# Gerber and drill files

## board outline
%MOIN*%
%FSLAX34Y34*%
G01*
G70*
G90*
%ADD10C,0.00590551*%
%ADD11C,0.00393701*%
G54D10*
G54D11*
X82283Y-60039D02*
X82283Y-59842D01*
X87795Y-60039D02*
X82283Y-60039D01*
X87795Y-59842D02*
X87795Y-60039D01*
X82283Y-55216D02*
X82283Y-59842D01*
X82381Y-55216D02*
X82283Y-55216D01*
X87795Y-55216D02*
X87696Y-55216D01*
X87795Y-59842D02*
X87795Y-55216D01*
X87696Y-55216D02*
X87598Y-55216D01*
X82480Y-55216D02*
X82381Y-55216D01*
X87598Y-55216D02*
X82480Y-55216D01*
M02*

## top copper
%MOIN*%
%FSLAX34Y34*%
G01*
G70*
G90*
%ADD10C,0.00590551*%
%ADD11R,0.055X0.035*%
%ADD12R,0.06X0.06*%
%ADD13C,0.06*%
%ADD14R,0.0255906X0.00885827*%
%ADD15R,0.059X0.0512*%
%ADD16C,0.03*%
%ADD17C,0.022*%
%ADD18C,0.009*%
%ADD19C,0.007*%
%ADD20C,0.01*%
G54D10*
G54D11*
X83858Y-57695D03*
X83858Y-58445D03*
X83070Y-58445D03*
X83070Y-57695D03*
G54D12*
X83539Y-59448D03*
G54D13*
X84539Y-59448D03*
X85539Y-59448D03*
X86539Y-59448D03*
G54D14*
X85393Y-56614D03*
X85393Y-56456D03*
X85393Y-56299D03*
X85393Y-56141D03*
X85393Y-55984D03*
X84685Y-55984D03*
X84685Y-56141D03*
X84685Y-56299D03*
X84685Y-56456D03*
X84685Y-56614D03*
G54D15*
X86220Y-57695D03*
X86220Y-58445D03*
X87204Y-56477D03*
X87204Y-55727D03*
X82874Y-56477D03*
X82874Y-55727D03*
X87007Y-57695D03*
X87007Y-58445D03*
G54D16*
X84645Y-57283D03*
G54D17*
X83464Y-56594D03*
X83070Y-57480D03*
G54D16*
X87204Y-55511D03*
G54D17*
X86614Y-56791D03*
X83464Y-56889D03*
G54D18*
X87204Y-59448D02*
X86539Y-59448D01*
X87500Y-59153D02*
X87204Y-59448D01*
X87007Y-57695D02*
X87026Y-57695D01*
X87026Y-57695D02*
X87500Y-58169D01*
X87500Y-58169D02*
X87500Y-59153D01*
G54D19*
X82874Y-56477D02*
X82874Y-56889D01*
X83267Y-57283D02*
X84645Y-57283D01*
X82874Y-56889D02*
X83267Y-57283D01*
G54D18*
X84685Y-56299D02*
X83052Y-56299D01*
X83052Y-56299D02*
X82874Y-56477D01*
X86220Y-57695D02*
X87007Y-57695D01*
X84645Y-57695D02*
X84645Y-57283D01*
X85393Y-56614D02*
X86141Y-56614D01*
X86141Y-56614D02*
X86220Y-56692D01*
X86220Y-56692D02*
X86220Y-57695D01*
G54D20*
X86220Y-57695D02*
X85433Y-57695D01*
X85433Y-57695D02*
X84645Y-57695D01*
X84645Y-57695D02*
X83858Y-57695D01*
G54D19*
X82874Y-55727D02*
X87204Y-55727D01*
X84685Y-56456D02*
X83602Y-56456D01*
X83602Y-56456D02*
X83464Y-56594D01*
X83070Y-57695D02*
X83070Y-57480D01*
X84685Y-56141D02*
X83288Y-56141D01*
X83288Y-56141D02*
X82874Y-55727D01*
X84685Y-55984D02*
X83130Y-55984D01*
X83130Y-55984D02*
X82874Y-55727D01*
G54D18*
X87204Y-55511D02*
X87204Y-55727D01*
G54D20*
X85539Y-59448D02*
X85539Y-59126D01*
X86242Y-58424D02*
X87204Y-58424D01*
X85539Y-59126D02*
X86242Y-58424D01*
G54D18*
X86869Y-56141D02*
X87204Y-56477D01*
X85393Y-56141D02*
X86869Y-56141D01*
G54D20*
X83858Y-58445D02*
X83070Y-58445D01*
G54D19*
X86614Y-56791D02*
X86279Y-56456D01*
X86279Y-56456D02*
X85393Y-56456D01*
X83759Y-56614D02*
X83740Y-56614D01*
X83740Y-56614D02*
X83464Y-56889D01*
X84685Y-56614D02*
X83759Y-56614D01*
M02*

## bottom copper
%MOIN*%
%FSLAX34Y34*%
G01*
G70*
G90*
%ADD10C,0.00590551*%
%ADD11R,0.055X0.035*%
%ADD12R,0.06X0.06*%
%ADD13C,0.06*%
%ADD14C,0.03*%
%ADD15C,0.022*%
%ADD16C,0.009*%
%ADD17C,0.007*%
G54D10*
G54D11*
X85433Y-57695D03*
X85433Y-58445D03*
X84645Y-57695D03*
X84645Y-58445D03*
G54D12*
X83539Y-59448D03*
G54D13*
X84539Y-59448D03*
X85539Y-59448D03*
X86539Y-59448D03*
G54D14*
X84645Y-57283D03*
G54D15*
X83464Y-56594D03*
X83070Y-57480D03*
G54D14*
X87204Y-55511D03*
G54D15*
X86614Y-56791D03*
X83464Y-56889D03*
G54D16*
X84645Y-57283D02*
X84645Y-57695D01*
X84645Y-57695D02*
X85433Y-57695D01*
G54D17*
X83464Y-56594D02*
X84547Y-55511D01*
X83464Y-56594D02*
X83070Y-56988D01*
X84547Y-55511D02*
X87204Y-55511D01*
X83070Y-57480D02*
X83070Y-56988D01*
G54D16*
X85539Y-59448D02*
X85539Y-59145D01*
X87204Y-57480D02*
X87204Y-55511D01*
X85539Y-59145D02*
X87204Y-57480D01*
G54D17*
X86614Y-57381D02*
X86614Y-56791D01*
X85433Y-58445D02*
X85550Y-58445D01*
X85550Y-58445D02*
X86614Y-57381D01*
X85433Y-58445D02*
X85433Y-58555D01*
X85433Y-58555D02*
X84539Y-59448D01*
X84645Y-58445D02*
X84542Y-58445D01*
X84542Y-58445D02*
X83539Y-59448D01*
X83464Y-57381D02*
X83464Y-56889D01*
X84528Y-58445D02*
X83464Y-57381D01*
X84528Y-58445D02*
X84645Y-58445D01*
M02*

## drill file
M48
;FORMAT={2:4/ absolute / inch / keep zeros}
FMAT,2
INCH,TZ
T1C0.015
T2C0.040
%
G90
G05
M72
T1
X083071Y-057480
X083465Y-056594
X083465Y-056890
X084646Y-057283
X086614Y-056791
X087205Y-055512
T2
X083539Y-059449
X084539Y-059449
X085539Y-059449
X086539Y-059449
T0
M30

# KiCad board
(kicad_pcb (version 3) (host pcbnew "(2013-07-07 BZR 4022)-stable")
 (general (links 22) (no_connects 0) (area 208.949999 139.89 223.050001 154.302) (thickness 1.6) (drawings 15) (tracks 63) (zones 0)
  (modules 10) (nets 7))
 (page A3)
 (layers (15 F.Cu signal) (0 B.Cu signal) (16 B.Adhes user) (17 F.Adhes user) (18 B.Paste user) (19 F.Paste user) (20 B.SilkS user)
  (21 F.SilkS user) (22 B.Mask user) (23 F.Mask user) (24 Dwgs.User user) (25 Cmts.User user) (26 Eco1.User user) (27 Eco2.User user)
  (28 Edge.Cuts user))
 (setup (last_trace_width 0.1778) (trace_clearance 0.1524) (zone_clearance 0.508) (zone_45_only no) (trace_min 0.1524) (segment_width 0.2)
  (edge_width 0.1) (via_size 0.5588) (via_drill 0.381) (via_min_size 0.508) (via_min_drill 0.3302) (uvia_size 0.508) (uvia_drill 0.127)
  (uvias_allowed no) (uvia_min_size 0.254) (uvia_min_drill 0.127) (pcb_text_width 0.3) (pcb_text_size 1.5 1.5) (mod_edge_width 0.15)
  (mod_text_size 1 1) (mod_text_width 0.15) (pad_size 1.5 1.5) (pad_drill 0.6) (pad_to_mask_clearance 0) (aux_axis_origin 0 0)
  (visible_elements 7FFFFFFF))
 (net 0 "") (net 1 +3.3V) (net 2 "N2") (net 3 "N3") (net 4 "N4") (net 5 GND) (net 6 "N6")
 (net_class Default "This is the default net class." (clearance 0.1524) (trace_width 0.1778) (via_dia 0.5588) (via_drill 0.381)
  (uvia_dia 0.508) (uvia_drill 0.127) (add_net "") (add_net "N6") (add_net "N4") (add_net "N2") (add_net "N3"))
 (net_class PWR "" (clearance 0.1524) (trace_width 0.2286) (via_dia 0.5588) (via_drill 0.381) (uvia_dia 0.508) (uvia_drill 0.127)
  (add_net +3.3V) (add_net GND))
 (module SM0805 (layer B.Cu) (at 217 147.5 270)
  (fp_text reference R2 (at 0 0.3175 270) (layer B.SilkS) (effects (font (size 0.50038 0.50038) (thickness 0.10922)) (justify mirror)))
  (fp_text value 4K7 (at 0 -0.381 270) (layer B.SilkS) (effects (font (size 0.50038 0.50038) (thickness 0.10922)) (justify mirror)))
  (pad 1 smd rect (at -0.9525 0 270) (size 0.889 1.397) (layers B.Cu B.Paste B.Mask) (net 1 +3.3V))
  (pad 2 smd rect (at 0.9525 0 270) (size 0.889 1.397) (layers B.Cu B.Paste B.Mask) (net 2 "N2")))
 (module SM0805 (layer B.Cu) (at 215 147.5 270)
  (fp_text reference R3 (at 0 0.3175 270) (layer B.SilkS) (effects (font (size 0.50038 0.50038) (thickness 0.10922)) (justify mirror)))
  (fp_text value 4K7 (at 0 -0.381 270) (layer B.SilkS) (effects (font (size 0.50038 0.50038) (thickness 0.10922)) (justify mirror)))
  (pad 1 smd rect (at -0.9525 0 270) (size 0.889 1.397) (layers B.Cu B.Paste B.Mask) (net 1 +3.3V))
  (pad 2 smd rect (at 0.9525 0 270) (size 0.889 1.397) (layers B.Cu B.Paste B.Mask) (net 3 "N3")))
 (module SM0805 (layer F.Cu) (at 213 147.5 270)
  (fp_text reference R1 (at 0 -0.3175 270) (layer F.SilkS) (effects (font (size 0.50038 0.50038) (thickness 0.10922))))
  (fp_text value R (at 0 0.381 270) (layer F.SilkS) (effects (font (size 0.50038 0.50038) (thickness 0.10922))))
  (pad 1 smd rect (at -0.9525 0 270) (size 0.889 1.397) (layers F.Cu F.Paste F.Mask) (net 1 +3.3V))
  (pad 2 smd rect (at 0.9525 0 270) (size 0.889 1.397) (layers F.Cu F.Paste F.Mask) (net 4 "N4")))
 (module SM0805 (layer F.Cu) (at 211 147.5 90)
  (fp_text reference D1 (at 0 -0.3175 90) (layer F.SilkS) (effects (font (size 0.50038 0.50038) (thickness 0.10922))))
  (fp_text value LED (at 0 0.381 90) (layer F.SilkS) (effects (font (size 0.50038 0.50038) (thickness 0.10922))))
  (pad 1 smd rect (at -0.9525 0 90) (size 0.889 1.397) (layers F.Cu F.Paste F.Mask) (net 4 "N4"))
  (pad 2 smd rect (at 0.9525 0 90) (size 0.889 1.397) (layers F.Cu F.Paste F.Mask) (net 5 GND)))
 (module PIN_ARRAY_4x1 (layer F.Cu) (at 216 151)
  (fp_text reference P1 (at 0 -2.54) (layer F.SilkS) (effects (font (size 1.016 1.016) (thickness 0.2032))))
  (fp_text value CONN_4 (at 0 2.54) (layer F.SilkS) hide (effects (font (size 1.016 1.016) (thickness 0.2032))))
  (pad 1 thru_hole rect (at -3.81 0) (size 1.524 1.524) (drill 1.016) (layers *.Cu *.Mask F.SilkS) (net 3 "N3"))
  (pad 2 thru_hole circle (at -1.27 0) (size 1.524 1.524) (drill 1.016) (layers *.Cu *.Mask F.SilkS) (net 2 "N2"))
  (pad 3 thru_hole circle (at 1.27 0) (size 1.524 1.524) (drill 1.016) (layers *.Cu *.Mask F.SilkS) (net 5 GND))
  (pad 4 thru_hole circle (at 3.81 0) (size 1.524 1.524) (drill 1.016) (layers *.Cu *.Mask F.SilkS) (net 1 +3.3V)))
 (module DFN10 (layer F.Cu) (at 216 143 180)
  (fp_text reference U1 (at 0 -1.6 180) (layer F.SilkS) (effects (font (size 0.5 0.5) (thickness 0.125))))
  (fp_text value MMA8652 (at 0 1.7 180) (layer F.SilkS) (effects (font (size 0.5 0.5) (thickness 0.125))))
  (pad 1 smd rect (at -0.9 -0.8 180) (size 0.65 0.225) (layers F.Cu F.Paste F.Mask) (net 1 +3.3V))
  (pad 2 smd rect (at -0.9 -0.4 180) (size 0.65 0.225) (layers F.Cu F.Paste F.Mask) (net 2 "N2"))
  (pad 3 smd rect (at -0.9 0 180) (size 0.65 0.225) (layers F.Cu F.Paste F.Mask))
  (pad 4 smd rect (at -0.9 0.4 180) (size 0.65 0.225) (layers F.Cu F.Paste F.Mask) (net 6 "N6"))
  (pad 5 smd rect (at -0.9 0.8 180) (size 0.65 0.225) (layers F.Cu F.Paste F.Mask))
  (pad 6 smd rect (at 0.9 0.8 180) (size 0.65 0.225) (layers F.Cu F.Paste F.Mask) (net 5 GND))
  (pad 7 smd rect (at 0.9 0.4 180) (size 0.65 0.225) (layers F.Cu F.Paste F.Mask) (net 5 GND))
  (pad 8 smd rect (at 0.9 0 180) (size 0.65 0.225) (layers F.Cu F.Paste F.Mask) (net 1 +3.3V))
  (pad 9 smd rect (at 0.9 -0.4 180) (size 0.65 0.225) (layers F.Cu F.Paste F.Mask) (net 5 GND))
  (pad 10 smd rect (at 0.9 -0.8 180) (size 0.65 0.225) (layers F.Cu F.Paste F.Mask) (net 3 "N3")))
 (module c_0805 (layer F.Cu) (at 219 147.5 90)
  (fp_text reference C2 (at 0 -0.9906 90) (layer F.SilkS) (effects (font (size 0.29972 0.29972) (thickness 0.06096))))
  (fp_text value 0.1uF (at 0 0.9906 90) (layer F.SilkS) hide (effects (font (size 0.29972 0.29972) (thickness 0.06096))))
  (pad 1 smd rect (at 0.9525 0 90) (size 1.30048 1.4986) (layers F.Cu F.Paste F.Mask) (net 1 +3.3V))
  (pad 2 smd rect (at -0.9525 0 90) (size 1.30048 1.4986) (layers F.Cu F.Paste F.Mask) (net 5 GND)))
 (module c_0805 (layer F.Cu) (at 221.5 142.5 270)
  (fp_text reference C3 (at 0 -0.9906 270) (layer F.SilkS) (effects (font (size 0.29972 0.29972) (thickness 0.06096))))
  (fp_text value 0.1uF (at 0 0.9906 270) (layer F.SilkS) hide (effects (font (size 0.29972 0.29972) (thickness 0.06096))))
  (pad 1 smd rect (at 0.9525 0 270) (size 1.30048 1.4986) (layers F.Cu F.Paste F.Mask) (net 6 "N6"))
  (pad 2 smd rect (at -0.9525 0 270) (size 1.30048 1.4986) (layers F.Cu F.Paste F.Mask) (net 5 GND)))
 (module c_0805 (layer F.Cu) (at 210.5 142.5 270)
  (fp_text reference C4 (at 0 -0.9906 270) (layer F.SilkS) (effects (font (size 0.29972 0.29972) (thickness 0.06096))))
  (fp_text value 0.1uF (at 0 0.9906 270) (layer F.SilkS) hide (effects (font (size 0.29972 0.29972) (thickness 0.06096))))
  (pad 1 smd rect (at 0.9525 0 270) (size 1.30048 1.4986) (layers F.Cu F.Paste F.Mask) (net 1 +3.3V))
  (pad 2 smd rect (at -0.9525 0 270) (size 1.30048 1.4986) (layers F.Cu F.Paste F.Mask) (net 5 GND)))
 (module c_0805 (layer F.Cu) (at 221 147.5 90)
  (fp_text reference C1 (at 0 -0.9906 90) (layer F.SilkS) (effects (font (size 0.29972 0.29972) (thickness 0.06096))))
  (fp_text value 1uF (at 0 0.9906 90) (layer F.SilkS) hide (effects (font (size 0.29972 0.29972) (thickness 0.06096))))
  (pad 1 smd rect (at 0.9525 0 90) (size 1.30048 1.4986) (layers F.Cu F.Paste F.Mask) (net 1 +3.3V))
  (pad 2 smd rect (at -0.9525 0 90) (size 1.30048 1.4986) (layers F.Cu F.Paste F.Mask) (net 5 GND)))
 (gr_line (start 209 152.5) (end 209 152) (angle 90) (layer Edge.Cuts) (width 0.1))
 (gr_line (start 223 152.5) (end 209 152.5) (angle 90) (layer Edge.Cuts) (width 0.1))
 (gr_line (start 223 152) (end 223 152.5) (angle 90) (layer Edge.Cuts) (width 0.1))
 (gr_line (start 209 140.25) (end 209 152) (angle 90) (layer Edge.Cuts) (width 0.1))
 (gr_line (start 209.25 140.25) (end 209 140.25) (angle 90) (layer Edge.Cuts) (width 0.1))
 (gr_line (start 223 140.25) (end 222.75 140.25) (angle 90) (layer Edge.Cuts) (width 0.1))
 (gr_line (start 223 152) (end 223 140.25) (angle 90) (layer Edge.Cuts) (width 0.1))
 (gr_line (start 222.75 140.25) (end 222.5 140.25) (angle 90) (layer Edge.Cuts) (width 0.1))
 (gr_line (start 209.5 140.25) (end 209.25 140.25) (angle 90) (layer Edge.Cuts) (width 0.1))
 (gr_line (start 222.5 140.25) (end 209.5 140.25) (angle 90) (layer Edge.Cuts) (width 0.1))
 (segment (start 221.5 151) (end 219.81 151) (width 0.2286) (layer F.Cu) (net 1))
 (segment (start 222.25 150.25) (end 221.5 151) (width 0.2286) (layer F.Cu) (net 1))
 (segment (start 221 146.5475) (end 221.0475 146.5475) (width 0.2286) (layer F.Cu) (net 1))
 (segment (start 221.0475 146.5475) (end 222.25 147.75) (width 0.2286) (layer F.Cu) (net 1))
 (segment (start 222.25 147.75) (end 222.25 150.25) (width 0.2286) (layer F.Cu) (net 1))
 (segment (start 210.5 143.4525) (end 210.5 144.5) (width 0.1778) (layer F.Cu) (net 1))
 (segment (start 211.5 145.5) (end 215 145.5) (width 0.1778) (layer F.Cu) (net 1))
 (segment (start 210.5 144.5) (end 211.5 145.5) (width 0.1778) (layer F.Cu) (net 1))
 (segment (start 215.1 143) (end 210.9525 143) (width 0.2286) (layer F.Cu) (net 1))
 (segment (start 210.9525 143) (end 210.5 143.4525) (width 0.2286) (layer F.Cu) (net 1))
 (segment (start 219 146.5475) (end 221 146.5475) (width 0.2286) (layer F.Cu) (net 1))
 (segment (start 215 146.5475) (end 215 145.5) (width 0.2286) (layer F.Cu) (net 1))
 (segment (start 215 145.5) (end 215 146.5475) (width 0.2286) (layer B.Cu) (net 1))
 (via (at 215 145.5) (size 0.762) (layers F.Cu B.Cu) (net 1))
 (segment (start 215 146.5475) (end 217 146.5475) (width 0.2286) (layer B.Cu) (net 1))
 (segment (start 216.9 143.8) (end 218.8 143.8) (width 0.2286) (layer F.Cu) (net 1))
 (segment (start 218.8 143.8) (end 219 144) (width 0.2286) (layer F.Cu) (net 1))
 (segment (start 219 144) (end 219 146.5475) (width 0.2286) (layer F.Cu) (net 1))
 (segment (start 219 146.5475) (end 217 146.5475) (width 0.254) (layer F.Cu) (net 1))
 (segment (start 217 146.5475) (end 215 146.5475) (width 0.254) (layer F.Cu) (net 1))
 (segment (start 215 146.5475) (end 213 146.5475) (width 0.254) (layer F.Cu) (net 1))
 (segment (start 210.5 141.5475) (end 221.5 141.5475) (width 0.1778) (layer F.Cu) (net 5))
 (segment (start 212 143.75) (end 214.75 141) (width 0.1778) (layer B.Cu) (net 5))
 (segment (start 215.1 143.4) (end 212.35 143.4) (width 0.1778) (layer F.Cu) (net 5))
 (segment (start 212 143.75) (end 211 144.75) (width 0.1778) (layer B.Cu) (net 5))
 (via (at 212 143.75) (size 0.5588) (layers F.Cu B.Cu) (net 5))
 (segment (start 212.35 143.4) (end 212 143.75) (width 0.1778) (layer F.Cu) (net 5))
 (segment (start 211 146.5475) (end 211 146) (width 0.1778) (layer F.Cu) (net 5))
 (segment (start 214.75 141) (end 221.5 141) (width 0.1778) (layer B.Cu) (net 5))
 (segment (start 211 146) (end 211 144.75) (width 0.1778) (layer B.Cu) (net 5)) (via (at 211 146) (size 0.5588) (layers F.Cu B.Cu) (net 5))
 (segment (start 215.1 142.6) (end 211.5525 142.6) (width 0.1778) (layer F.Cu) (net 5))
 (segment (start 211.5525 142.6) (end 210.5 141.5475) (width 0.1778) (layer F.Cu) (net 5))
 (segment (start 215.1 142.2) (end 211.1525 142.2) (width 0.1778) (layer F.Cu) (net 5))
 (segment (start 211.1525 142.2) (end 210.5 141.5475) (width 0.1778) (layer F.Cu) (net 5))
 (segment (start 217.27 151) (end 217.27 150.23) (width 0.2286) (layer B.Cu) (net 5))
 (segment (start 221.5 141) (end 221.5 141.5475) (width 0.2286) (layer F.Cu) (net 5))
 (via (at 221.5 141) (size 0.762) (layers F.Cu B.Cu) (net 5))
 (segment (start 221.5 146) (end 221.5 141) (width 0.2286) (layer B.Cu) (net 5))
 (segment (start 217.27 150.23) (end 221.5 146) (width 0.2286) (layer B.Cu) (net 5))
 (segment (start 217.27 151) (end 217.27 150.1825) (width 0.254) (layer F.Cu) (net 5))
 (segment (start 219.0555 148.397) (end 221.5 148.397) (width 0.254) (layer F.Cu) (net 5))
 (segment (start 217.27 150.1825) (end 219.0555 148.397) (width 0.254) (layer F.Cu) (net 5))
 (segment (start 220.6475 142.6) (end 221.5 143.4525) (width 0.2286) (layer F.Cu) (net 6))
 (segment (start 216.9 142.6) (end 220.6475 142.6) (width 0.2286) (layer F.Cu) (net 6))
 (segment (start 213 148.4525) (end 211 148.4525) (width 0.254) (layer F.Cu) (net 4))
 (segment (start 220 144.25) (end 219.15 143.4) (width 0.1778) (layer F.Cu) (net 2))
 (segment (start 220 145.75) (end 220 144.25) (width 0.1778) (layer B.Cu) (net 2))
 (via (at 220 144.25) (size 0.5588) (layers F.Cu B.Cu) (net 2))
 (segment (start 217 148.4525) (end 217.2975 148.4525) (width 0.1778) (layer B.Cu) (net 2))
 (segment (start 217.2975 148.4525) (end 220 145.75) (width 0.1778) (layer B.Cu) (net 2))
 (segment (start 219.15 143.4) (end 216.9 143.4) (width 0.1778) (layer F.Cu) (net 2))
 (segment (start 217 148.4525) (end 217 148.73) (width 0.1778) (layer B.Cu) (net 2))
 (segment (start 217 148.73) (end 214.73 151) (width 0.1778) (layer B.Cu) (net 2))
 (segment (start 215 148.4525) (end 214.7375 148.4525) (width 0.1778) (layer B.Cu) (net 3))
 (segment (start 214.7375 148.4525) (end 212.19 151) (width 0.1778) (layer B.Cu) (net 3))
 (segment (start 212 145.75) (end 212 144.5) (width 0.1778) (layer B.Cu) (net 3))
 (segment (start 212.75 143.8) (end 212.7 143.8) (width 0.1778) (layer F.Cu) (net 3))
 (segment (start 212.7 143.8) (end 212 144.5) (width 0.1778) (layer F.Cu) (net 3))
 (segment (start 215.1 143.8) (end 212.75 143.8) (width 0.1778) (layer F.Cu) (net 3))
 (via (at 212 144.5) (size 0.5588) (layers F.Cu B.Cu) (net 3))
 (segment (start 214.7025 148.4525) (end 212 145.75) (width 0.1778) (layer B.Cu) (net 3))
 (segment (start 214.7025 148.4525) (end 215 148.4525) (width 0.1778) (layer B.Cu) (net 3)))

